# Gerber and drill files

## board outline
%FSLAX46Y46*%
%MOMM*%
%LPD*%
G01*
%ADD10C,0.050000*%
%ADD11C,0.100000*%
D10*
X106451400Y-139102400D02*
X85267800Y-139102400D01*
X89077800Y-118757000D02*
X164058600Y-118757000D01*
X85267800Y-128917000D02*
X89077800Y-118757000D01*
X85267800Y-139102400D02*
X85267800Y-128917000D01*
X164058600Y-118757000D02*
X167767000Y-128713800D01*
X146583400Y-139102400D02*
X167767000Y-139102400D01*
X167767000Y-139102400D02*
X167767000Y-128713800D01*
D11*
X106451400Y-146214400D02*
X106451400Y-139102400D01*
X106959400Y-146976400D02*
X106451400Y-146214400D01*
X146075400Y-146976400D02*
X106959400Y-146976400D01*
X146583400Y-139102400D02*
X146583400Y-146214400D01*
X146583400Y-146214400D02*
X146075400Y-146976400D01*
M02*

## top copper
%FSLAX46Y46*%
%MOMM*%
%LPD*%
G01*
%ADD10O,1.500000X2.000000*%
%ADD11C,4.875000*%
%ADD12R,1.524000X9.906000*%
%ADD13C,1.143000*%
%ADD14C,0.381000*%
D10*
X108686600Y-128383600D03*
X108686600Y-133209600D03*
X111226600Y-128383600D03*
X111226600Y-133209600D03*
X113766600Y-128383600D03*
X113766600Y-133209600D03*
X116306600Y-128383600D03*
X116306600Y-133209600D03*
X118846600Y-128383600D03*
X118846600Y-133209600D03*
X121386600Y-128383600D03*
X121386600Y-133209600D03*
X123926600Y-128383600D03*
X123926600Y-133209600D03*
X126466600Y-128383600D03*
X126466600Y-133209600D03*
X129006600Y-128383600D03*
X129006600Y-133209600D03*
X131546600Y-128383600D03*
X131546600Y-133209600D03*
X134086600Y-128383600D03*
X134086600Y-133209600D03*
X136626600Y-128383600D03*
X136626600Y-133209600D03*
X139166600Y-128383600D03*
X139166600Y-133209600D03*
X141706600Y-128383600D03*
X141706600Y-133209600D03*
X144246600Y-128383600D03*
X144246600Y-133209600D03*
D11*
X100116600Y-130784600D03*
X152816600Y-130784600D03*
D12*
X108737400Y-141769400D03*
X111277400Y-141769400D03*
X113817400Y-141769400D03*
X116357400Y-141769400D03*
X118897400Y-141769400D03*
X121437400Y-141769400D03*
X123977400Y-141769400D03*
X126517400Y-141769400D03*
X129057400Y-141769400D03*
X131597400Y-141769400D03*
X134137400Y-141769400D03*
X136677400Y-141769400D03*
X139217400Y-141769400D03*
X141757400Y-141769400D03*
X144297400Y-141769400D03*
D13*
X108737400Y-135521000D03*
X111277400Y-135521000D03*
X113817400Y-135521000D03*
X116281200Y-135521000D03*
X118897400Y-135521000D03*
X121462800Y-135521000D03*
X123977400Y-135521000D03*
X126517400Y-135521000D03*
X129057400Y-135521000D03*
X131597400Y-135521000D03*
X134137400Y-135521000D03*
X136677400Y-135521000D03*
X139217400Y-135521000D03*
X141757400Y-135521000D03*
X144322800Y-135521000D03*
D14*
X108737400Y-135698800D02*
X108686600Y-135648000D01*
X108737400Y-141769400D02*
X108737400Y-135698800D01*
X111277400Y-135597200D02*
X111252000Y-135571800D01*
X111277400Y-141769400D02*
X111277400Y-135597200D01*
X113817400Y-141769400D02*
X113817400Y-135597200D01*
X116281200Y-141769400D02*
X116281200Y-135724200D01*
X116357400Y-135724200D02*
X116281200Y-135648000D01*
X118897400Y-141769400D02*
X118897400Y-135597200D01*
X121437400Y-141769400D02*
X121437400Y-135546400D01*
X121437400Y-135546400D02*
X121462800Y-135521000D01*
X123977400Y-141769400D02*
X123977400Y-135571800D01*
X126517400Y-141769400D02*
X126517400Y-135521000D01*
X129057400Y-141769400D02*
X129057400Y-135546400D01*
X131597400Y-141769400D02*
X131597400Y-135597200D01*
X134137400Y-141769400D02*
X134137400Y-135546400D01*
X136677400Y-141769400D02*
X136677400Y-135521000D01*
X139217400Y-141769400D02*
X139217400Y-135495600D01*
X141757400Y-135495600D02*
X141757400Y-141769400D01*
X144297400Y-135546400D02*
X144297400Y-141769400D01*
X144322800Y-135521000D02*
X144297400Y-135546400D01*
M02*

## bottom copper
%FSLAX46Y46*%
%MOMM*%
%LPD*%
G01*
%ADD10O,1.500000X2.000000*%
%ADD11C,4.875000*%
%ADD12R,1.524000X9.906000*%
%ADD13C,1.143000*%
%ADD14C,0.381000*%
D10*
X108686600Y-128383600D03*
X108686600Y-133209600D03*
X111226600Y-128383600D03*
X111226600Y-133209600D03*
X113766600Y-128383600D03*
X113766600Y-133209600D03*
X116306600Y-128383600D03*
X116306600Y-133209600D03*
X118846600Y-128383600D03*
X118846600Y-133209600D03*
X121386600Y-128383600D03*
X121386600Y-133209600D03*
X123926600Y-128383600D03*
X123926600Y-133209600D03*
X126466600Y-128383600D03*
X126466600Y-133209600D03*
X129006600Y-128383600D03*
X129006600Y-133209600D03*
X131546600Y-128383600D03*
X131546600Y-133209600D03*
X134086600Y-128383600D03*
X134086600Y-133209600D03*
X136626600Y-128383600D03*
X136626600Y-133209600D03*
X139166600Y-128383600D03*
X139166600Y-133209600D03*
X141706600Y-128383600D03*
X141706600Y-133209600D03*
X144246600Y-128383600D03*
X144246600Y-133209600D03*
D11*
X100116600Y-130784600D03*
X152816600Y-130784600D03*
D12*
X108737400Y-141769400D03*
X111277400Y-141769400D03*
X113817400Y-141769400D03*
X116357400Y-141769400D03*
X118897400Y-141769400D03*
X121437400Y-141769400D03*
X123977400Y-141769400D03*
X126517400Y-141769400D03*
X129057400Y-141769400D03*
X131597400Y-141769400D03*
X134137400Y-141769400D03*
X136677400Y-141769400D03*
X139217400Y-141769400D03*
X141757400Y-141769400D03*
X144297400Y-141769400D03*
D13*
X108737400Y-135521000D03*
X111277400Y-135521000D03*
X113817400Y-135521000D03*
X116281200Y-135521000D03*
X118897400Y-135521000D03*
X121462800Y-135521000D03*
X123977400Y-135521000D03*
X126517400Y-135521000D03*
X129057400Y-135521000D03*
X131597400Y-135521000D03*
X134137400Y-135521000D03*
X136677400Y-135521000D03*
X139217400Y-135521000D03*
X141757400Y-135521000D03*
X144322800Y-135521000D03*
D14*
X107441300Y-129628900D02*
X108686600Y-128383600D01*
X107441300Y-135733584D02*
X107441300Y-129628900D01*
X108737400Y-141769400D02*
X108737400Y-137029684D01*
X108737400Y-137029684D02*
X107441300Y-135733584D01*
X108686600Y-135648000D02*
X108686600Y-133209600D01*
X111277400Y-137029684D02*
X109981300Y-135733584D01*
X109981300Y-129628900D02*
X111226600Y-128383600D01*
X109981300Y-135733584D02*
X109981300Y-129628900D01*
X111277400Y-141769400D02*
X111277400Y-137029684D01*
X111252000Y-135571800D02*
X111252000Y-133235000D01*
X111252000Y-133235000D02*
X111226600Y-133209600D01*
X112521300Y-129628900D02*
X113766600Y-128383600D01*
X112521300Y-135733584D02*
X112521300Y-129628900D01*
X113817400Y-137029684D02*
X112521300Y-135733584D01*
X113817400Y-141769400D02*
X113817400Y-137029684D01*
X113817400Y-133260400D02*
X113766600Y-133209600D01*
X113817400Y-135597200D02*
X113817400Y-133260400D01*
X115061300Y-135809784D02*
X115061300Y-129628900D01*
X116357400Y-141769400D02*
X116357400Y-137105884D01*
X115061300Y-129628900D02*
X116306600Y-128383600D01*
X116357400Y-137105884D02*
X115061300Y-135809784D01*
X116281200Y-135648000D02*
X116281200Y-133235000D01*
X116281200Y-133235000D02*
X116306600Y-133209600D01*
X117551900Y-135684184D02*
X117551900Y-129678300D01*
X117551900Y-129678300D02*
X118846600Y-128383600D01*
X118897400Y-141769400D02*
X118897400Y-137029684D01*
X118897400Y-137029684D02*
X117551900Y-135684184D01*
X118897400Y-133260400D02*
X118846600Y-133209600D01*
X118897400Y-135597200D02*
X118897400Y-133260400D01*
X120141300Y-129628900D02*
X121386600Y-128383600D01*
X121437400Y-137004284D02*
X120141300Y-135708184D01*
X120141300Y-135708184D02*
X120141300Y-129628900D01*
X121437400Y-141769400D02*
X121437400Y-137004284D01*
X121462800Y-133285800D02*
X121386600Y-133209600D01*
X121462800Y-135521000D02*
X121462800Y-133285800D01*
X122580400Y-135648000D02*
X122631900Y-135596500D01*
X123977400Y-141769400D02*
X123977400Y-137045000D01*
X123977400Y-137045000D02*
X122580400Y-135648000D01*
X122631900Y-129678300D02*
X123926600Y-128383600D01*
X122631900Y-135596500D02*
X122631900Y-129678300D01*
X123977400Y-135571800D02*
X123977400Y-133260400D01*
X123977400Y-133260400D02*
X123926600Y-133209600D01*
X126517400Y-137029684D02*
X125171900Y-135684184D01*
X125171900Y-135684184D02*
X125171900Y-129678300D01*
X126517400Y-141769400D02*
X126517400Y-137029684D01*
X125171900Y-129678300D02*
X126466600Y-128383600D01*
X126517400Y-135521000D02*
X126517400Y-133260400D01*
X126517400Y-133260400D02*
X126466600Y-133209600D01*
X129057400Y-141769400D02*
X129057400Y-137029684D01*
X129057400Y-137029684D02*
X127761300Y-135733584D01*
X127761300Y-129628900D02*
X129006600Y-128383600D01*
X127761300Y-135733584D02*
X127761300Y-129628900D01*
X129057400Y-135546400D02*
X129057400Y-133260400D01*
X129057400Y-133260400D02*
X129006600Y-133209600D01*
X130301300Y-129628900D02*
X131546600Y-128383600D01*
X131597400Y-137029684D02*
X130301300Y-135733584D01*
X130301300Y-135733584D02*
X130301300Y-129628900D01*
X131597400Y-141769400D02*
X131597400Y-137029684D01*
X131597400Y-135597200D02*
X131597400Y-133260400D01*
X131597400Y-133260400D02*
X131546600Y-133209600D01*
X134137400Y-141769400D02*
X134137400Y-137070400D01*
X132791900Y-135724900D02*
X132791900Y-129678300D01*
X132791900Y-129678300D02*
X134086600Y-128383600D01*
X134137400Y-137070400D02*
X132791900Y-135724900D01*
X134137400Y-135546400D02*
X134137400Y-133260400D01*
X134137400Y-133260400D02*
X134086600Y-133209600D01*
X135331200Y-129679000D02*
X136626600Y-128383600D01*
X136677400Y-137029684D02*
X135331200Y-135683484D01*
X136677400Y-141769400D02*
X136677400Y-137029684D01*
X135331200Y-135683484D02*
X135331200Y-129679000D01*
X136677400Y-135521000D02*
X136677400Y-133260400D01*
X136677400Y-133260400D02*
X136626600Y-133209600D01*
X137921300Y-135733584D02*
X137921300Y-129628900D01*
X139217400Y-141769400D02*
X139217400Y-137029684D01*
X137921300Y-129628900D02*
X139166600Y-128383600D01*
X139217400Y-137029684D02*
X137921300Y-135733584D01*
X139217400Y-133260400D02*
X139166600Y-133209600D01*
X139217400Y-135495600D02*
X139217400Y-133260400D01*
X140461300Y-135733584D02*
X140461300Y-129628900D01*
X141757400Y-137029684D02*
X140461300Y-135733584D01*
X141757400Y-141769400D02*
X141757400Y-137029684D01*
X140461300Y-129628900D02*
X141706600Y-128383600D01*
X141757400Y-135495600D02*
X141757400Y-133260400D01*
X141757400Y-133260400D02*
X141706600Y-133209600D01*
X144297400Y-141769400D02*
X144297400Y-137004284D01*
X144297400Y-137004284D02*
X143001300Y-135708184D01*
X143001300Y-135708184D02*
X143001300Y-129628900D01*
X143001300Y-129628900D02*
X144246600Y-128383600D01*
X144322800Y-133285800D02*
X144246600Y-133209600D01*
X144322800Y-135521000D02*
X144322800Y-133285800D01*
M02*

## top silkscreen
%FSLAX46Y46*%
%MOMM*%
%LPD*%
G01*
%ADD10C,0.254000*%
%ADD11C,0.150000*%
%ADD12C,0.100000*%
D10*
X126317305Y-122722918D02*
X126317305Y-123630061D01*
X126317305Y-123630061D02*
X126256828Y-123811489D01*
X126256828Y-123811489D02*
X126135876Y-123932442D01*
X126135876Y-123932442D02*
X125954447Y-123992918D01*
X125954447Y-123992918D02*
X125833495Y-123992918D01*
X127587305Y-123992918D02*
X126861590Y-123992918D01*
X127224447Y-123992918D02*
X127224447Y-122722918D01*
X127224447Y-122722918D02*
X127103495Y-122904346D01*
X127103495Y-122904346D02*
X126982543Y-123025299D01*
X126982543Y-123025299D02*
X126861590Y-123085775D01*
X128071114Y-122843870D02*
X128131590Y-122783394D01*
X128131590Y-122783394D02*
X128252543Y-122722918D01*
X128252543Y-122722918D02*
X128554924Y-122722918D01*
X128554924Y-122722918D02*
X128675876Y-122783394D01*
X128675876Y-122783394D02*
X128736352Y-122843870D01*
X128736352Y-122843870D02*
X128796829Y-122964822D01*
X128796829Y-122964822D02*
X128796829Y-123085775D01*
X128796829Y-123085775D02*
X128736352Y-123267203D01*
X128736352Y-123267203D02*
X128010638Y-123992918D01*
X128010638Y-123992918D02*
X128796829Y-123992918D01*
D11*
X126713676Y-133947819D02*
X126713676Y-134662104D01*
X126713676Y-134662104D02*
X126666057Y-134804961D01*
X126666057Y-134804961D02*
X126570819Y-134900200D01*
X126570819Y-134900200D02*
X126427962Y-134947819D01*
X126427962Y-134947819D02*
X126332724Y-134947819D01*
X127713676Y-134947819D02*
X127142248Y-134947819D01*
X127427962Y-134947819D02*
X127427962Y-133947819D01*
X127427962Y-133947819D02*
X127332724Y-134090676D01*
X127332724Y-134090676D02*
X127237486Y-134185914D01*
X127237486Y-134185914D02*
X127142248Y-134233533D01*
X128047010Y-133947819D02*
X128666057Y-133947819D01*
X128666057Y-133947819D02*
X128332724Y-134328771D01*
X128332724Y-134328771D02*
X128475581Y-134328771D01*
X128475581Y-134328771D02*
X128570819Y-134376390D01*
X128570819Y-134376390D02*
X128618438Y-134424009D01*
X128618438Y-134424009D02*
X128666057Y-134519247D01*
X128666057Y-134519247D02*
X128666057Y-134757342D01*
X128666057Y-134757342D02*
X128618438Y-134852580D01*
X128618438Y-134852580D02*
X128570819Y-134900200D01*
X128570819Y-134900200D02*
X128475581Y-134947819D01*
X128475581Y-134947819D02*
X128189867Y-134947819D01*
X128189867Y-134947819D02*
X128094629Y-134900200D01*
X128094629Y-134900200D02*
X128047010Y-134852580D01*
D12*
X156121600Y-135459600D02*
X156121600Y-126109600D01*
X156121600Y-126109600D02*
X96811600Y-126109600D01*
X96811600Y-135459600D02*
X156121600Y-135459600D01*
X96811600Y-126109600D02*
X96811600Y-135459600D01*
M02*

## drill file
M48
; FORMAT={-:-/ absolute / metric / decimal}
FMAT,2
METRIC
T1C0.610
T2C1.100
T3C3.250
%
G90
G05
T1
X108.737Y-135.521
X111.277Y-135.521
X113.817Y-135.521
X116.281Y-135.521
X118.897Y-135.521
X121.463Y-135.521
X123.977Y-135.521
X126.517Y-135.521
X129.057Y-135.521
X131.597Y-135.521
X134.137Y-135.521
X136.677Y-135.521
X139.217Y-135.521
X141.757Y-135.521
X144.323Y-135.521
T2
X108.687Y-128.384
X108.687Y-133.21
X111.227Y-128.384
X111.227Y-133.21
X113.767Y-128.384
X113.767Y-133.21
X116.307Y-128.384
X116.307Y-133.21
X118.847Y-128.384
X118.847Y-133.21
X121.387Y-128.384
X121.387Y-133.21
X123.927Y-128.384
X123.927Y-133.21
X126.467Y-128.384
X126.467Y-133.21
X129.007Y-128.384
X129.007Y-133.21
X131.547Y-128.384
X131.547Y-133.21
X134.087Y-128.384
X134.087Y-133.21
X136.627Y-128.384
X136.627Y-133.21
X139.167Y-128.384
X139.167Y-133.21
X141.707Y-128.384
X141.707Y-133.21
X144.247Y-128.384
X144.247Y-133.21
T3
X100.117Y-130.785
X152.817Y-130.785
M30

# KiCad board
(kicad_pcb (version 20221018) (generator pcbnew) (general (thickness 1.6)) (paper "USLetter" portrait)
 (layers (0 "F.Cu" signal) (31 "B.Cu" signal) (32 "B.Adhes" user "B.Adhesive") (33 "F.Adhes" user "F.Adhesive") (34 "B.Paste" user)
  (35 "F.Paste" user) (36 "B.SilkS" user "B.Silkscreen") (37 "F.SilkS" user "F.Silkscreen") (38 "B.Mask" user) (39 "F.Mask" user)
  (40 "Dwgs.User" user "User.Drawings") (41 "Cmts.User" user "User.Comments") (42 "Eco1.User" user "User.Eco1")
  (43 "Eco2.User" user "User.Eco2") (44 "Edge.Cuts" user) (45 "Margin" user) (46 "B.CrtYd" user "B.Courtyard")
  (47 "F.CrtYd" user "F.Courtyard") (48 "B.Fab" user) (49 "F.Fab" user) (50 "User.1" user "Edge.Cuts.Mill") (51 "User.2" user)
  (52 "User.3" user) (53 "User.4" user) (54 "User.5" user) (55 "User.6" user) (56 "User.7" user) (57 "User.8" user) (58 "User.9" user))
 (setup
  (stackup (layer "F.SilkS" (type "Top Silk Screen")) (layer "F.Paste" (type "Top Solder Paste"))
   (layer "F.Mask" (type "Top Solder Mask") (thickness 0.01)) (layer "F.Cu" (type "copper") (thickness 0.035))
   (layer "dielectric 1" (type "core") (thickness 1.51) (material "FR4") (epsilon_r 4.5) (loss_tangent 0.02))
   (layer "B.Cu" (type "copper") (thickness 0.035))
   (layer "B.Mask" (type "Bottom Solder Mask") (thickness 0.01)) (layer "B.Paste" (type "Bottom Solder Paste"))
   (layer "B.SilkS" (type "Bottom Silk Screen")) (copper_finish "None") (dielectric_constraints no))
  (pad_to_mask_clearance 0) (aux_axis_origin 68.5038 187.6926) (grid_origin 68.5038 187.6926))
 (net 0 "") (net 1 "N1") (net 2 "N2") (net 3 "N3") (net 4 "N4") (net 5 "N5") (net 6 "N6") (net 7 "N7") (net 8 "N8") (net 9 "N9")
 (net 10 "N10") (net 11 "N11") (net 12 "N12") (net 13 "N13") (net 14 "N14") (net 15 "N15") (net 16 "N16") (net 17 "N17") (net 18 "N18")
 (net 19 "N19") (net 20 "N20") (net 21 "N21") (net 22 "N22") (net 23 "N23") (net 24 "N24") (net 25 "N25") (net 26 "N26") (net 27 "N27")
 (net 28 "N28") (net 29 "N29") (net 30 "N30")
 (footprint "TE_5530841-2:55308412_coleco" (layer "F.Cu") (at 108.6866 133.2096 180)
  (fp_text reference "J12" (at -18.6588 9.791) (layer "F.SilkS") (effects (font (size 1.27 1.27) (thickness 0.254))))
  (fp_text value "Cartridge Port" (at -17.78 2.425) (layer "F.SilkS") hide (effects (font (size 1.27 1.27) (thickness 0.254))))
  (fp_line (start -47.435 -2.25) (end -47.435 7.1) (stroke (width 0.1) (type solid)) (layer "F.SilkS"))
  (fp_line (start -47.435 7.1) (end 11.875 7.1) (stroke (width 0.1) (type solid)) (layer "F.SilkS"))
  (fp_line (start 11.875 -2.25) (end -47.435 -2.25) (stroke (width 0.1) (type solid)) (layer "F.SilkS"))
  (fp_line (start 11.875 7.1) (end 11.875 -2.25) (stroke (width 0.1) (type solid)) (layer "F.SilkS"))
  (pad "1" thru_hole oval (at 0 4.826 180) (size 1.5 2) (drill 1.1) (layers "*.Cu" "*.Mask") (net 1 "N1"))
  (pad "2" thru_hole oval (at 0 0 180) (size 1.5 2) (drill 1.1) (layers "*.Cu" "*.Mask") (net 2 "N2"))
  (pad "3" thru_hole oval (at -2.54 4.826 180) (size 1.5 2) (drill 1.1) (layers "*.Cu" "*.Mask") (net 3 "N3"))
  (pad "4" thru_hole oval (at -2.54 0 180) (size 1.5 2) (drill 1.1) (layers "*.Cu" "*.Mask") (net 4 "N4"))
  (pad "5" thru_hole oval (at -5.08 4.826 180) (size 1.5 2) (drill 1.1) (layers "*.Cu" "*.Mask") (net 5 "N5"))
  (pad "6" thru_hole oval (at -5.08 0 180) (size 1.5 2) (drill 1.1) (layers "*.Cu" "*.Mask") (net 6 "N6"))
  (pad "7" thru_hole oval (at -7.62 4.826 180) (size 1.5 2) (drill 1.1) (layers "*.Cu" "*.Mask") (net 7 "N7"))
  (pad "8" thru_hole oval (at -7.62 0 180) (size 1.5 2) (drill 1.1) (layers "*.Cu" "*.Mask") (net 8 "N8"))
  (pad "9" thru_hole oval (at -10.16 4.826 180) (size 1.5 2) (drill 1.1) (layers "*.Cu" "*.Mask") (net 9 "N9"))
  (pad "10" thru_hole oval (at -10.16 0 180) (size 1.5 2) (drill 1.1) (layers "*.Cu" "*.Mask") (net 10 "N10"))
  (pad "11" thru_hole oval (at -12.7 4.826 180) (size 1.5 2) (drill 1.1) (layers "*.Cu" "*.Mask") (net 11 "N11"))
  (pad "12" thru_hole oval (at -12.7 0 180) (size 1.5 2) (drill 1.1) (layers "*.Cu" "*.Mask") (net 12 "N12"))
  (pad "13" thru_hole oval (at -15.24 4.826 180) (size 1.5 2) (drill 1.1) (layers "*.Cu" "*.Mask") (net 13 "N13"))
  (pad "14" thru_hole oval (at -15.24 0 180) (size 1.5 2) (drill 1.1) (layers "*.Cu" "*.Mask") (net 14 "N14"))
  (pad "15" thru_hole oval (at -17.78 4.826 180) (size 1.5 2) (drill 1.1) (layers "*.Cu" "*.Mask") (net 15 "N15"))
  (pad "16" thru_hole oval (at -17.78 0 180) (size 1.5 2) (drill 1.1) (layers "*.Cu" "*.Mask") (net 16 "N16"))
  (pad "17" thru_hole oval (at -20.32 4.826 180) (size 1.5 2) (drill 1.1) (layers "*.Cu" "*.Mask") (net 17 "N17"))
  (pad "18" thru_hole oval (at -20.32 0 180) (size 1.5 2) (drill 1.1) (layers "*.Cu" "*.Mask") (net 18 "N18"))
  (pad "19" thru_hole oval (at -22.86 4.826 180) (size 1.5 2) (drill 1.1) (layers "*.Cu" "*.Mask") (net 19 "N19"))
  (pad "20" thru_hole oval (at -22.86 0 180) (size 1.5 2) (drill 1.1) (layers "*.Cu" "*.Mask") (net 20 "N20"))
  (pad "21" thru_hole oval (at -25.4 4.826 180) (size 1.5 2) (drill 1.1) (layers "*.Cu" "*.Mask") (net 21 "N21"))
  (pad "22" thru_hole oval (at -25.4 0 180) (size 1.5 2) (drill 1.1) (layers "*.Cu" "*.Mask") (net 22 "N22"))
  (pad "23" thru_hole oval (at -27.94 4.826 180) (size 1.5 2) (drill 1.1) (layers "*.Cu" "*.Mask") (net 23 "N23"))
  (pad "24" thru_hole oval (at -27.94 0 180) (size 1.5 2) (drill 1.1) (layers "*.Cu" "*.Mask") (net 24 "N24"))
  (pad "25" thru_hole oval (at -30.48 4.826 180) (size 1.5 2) (drill 1.1) (layers "*.Cu" "*.Mask") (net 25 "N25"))
  (pad "26" thru_hole oval (at -30.48 0 180) (size 1.5 2) (drill 1.1) (layers "*.Cu" "*.Mask") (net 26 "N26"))
  (pad "27" thru_hole oval (at -33.02 4.826 180) (size 1.5 2) (drill 1.1) (layers "*.Cu" "*.Mask") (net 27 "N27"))
  (pad "28" thru_hole oval (at -33.02 0 180) (size 1.5 2) (drill 1.1) (layers "*.Cu" "*.Mask") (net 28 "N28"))
  (pad "29" thru_hole oval (at -35.56 4.826 180) (size 1.5 2) (drill 1.1) (layers "*.Cu" "*.Mask") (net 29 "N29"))
  (pad "30" thru_hole oval (at -35.56 0 180) (size 1.5 2) (drill 1.1) (layers "*.Cu" "*.Mask") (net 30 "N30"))
  (pad "MH1" thru_hole circle (at 8.57 2.425 180) (size 4.875 4.875) (drill 3.25) (layers "*.Cu" "*.Mask"))
  (pad "MH2" thru_hole circle (at -44.13 2.425 180) (size 4.875 4.875) (drill 3.25) (layers "*.Cu" "*.Mask")))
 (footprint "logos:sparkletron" (layer "F.Cu") (at 138.3842 226.960062)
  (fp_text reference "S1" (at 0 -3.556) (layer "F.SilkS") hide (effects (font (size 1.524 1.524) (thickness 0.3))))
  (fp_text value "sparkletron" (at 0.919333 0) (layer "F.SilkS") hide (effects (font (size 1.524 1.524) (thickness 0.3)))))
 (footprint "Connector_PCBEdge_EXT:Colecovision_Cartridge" (layer "F.Cu") (at 104.9274 143.6744)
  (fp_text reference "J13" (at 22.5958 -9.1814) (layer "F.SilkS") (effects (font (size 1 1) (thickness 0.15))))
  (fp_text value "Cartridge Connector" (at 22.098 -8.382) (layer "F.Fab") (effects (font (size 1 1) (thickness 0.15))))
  (fp_line (start 1.524 2.54) (end 1.524 -4.572) (stroke (width 0.1) (type solid)) (layer "Edge.Cuts"))
  (fp_line (start 2.032 3.302) (end 1.524 2.54) (stroke (width 0.1) (type solid)) (layer "Edge.Cuts"))
  (fp_line (start 41.148 3.302) (end 2.032 3.302) (stroke (width 0.1) (type solid)) (layer "Edge.Cuts"))
  (fp_line (start 41.656 -4.572) (end 41.656 2.54) (stroke (width 0.1) (type solid)) (layer "Edge.Cuts"))
  (fp_line (start 41.656 2.54) (end 41.148 3.302) (stroke (width 0.1) (type solid)) (layer "Edge.Cuts"))
  (pad "1" connect rect (at 3.81 -1.905) (size 1.524 9.906) (layers "B.Cu" "B.Mask") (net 1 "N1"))
  (pad "2" connect rect (at 3.81 -1.905) (size 1.524 9.906) (layers "F.Cu" "F.Mask") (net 2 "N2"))
  (pad "3" connect rect (at 6.35 -1.905) (size 1.524 9.906) (layers "B.Cu" "B.Mask") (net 3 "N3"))
  (pad "4" connect rect (at 6.35 -1.905) (size 1.524 9.906) (layers "F.Cu" "F.Mask") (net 4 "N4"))
  (pad "5" connect rect (at 8.89 -1.905) (size 1.524 9.906) (layers "B.Cu" "B.Mask") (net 5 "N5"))
  (pad "6" connect rect (at 8.89 -1.905) (size 1.524 9.906) (layers "F.Cu" "F.Mask") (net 6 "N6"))
  (pad "7" connect rect (at 11.43 -1.905) (size 1.524 9.906) (layers "B.Cu" "B.Mask") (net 7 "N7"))
  (pad "8" connect rect (at 11.43 -1.905) (size 1.524 9.906) (layers "F.Cu" "F.Mask") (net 8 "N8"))
  (pad "9" connect rect (at 13.97 -1.905) (size 1.524 9.906) (layers "B.Cu" "B.Mask") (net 9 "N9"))
  (pad "10" connect rect (at 13.97 -1.905) (size 1.524 9.906) (layers "F.Cu" "F.Mask") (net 10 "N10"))
  (pad "11" connect rect (at 16.51 -1.905) (size 1.524 9.906) (layers "B.Cu" "B.Mask") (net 11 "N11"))
  (pad "12" connect rect (at 16.51 -1.905) (size 1.524 9.906) (layers "F.Cu" "F.Mask") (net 12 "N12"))
  (pad "13" connect rect (at 19.05 -1.905) (size 1.524 9.906) (layers "B.Cu" "B.Mask") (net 13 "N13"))
  (pad "14" connect rect (at 19.05 -1.905) (size 1.524 9.906) (layers "F.Cu" "F.Mask") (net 14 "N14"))
  (pad "15" connect rect (at 21.59 -1.905) (size 1.524 9.906) (layers "B.Cu" "B.Mask") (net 15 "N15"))
  (pad "16" connect rect (at 21.59 -1.905) (size 1.524 9.906) (layers "F.Cu" "F.Mask") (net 16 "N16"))
  (pad "17" connect rect (at 24.13 -1.905) (size 1.524 9.906) (layers "B.Cu" "B.Mask") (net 17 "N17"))
  (pad "18" connect rect (at 24.13 -1.905) (size 1.524 9.906) (layers "F.Cu" "F.Mask") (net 18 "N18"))
  (pad "19" connect rect (at 26.67 -1.905) (size 1.524 9.906) (layers "B.Cu" "B.Mask") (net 19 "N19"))
  (pad "20" connect rect (at 26.67 -1.905) (size 1.524 9.906) (layers "F.Cu" "F.Mask") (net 20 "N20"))
  (pad "21" connect rect (at 29.21 -1.905) (size 1.524 9.906) (layers "B.Cu" "B.Mask") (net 21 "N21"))
  (pad "22" connect rect (at 29.21 -1.905) (size 1.524 9.906) (layers "F.Cu" "F.Mask") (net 22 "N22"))
  (pad "23" connect rect (at 31.75 -1.905) (size 1.524 9.906) (layers "B.Cu" "B.Mask") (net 23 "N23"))
  (pad "24" connect rect (at 31.75 -1.905) (size 1.524 9.906) (layers "F.Cu" "F.Mask") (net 24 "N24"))
  (pad "25" connect rect (at 34.29 -1.905) (size 1.524 9.906) (layers "B.Cu" "B.Mask") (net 25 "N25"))
  (pad "26" connect rect (at 34.29 -1.905) (size 1.524 9.906) (layers "F.Cu" "F.Mask") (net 26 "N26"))
  (pad "27" connect rect (at 36.83 -1.905) (size 1.524 9.906) (layers "B.Cu" "B.Mask") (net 27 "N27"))
  (pad "28" connect rect (at 36.83 -1.905) (size 1.524 9.906) (layers "F.Cu" "F.Mask") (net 28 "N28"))
  (pad "29" connect rect (at 39.37 -1.905) (size 1.524 9.906) (layers "B.Cu" "B.Mask") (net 29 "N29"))
  (pad "30" connect rect (at 39.37 -1.905) (size 1.524 9.906) (layers "F.Cu" "F.Mask") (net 30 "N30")))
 (gr_line (start 106.4514 139.1024) (end 85.2678 139.1024) (stroke (width 0.05) (type default)) (layer "Edge.Cuts"))
 (gr_line (start 89.0778 118.757) (end 164.0586 118.757) (stroke (width 0.05) (type default)) (layer "Edge.Cuts"))
 (gr_line (start 85.2678 128.917) (end 89.0778 118.757) (stroke (width 0.05) (type default)) (layer "Edge.Cuts"))
 (gr_line (start 85.2678 139.1024) (end 85.2678 128.917) (stroke (width 0.05) (type default)) (layer "Edge.Cuts"))
 (gr_line (start 164.0586 118.757) (end 167.767 128.7138) (stroke (width 0.05) (type default)) (layer "Edge.Cuts"))
 (gr_line (start 146.5834 139.1024) (end 167.767 139.1024) (stroke (width 0.05) (type default)) (layer "Edge.Cuts"))
 (gr_line (start 167.767 139.1024) (end 167.767 128.7138) (stroke (width 0.05) (type default)) (layer "Edge.Cuts"))
 (segment (start 107.4413 129.6289) (end 108.6866 128.3836) (width 0.381) (layer "B.Cu") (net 1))
 (segment (start 107.4413 135.733584) (end 107.4413 129.6289) (width 0.381) (layer "B.Cu") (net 1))
 (segment (start 108.7374 141.7694) (end 108.7374 137.029684) (width 0.381) (layer "B.Cu") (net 1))
 (segment (start 108.7374 137.029684) (end 107.4413 135.733584) (width 0.381) (layer "B.Cu") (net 1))
 (segment (start 108.7374 135.6988) (end 108.6866 135.648) (width 0.381) (layer "F.Cu") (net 2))
 (segment (start 108.7374 141.7694) (end 108.7374 135.6988) (width 0.381) (layer "F.Cu") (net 2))
 (via (at 108.7374 135.521) (size 1.143) (drill 0.6096) (layers "F.Cu" "B.Cu") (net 2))
 (segment (start 108.6866 135.648) (end 108.6866 133.2096) (width 0.381) (layer "B.Cu") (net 2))
 (segment (start 111.2774 137.029684) (end 109.9813 135.733584) (width 0.381) (layer "B.Cu") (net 3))
 (segment (start 109.9813 129.6289) (end 111.2266 128.3836) (width 0.381) (layer "B.Cu") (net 3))
 (segment (start 109.9813 135.733584) (end 109.9813 129.6289) (width 0.381) (layer "B.Cu") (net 3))
 (segment (start 111.2774 141.7694) (end 111.2774 137.029684) (width 0.381) (layer "B.Cu") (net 3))
 (segment (start 111.2774 135.5972) (end 111.252 135.5718) (width 0.381) (layer "F.Cu") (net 4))
 (segment (start 111.2774 141.7694) (end 111.2774 135.5972) (width 0.381) (layer "F.Cu") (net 4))
 (via (at 111.2774 135.521) (size 1.143) (drill 0.6096) (layers "F.Cu" "B.Cu") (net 4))
 (segment (start 111.252 135.5718) (end 111.252 133.235) (width 0.381) (layer "B.Cu") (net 4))
 (segment (start 111.252 133.235) (end 111.2266 133.2096) (width 0.381) (layer "B.Cu") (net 4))
 (segment (start 112.5213 129.6289) (end 113.7666 128.3836) (width 0.381) (layer "B.Cu") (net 5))
 (segment (start 112.5213 135.733584) (end 112.5213 129.6289) (width 0.381) (layer "B.Cu") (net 5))
 (segment (start 113.8174 137.029684) (end 112.5213 135.733584) (width 0.381) (layer "B.Cu") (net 5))
 (segment (start 113.8174 141.7694) (end 113.8174 137.029684) (width 0.381) (layer "B.Cu") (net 5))
 (segment (start 113.8174 141.7694) (end 113.8174 135.5972) (width 0.381) (layer "F.Cu") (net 6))
 (via (at 113.8174 135.521) (size 1.143) (drill 0.6096) (layers "F.Cu" "B.Cu") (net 6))
 (segment (start 113.8174 133.2604) (end 113.7666 133.2096) (width 0.381) (layer "B.Cu") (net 6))
 (segment (start 113.8174 135.5972) (end 113.8174 133.2604) (width 0.381) (layer "B.Cu") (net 6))
 (segment (start 115.0613 135.809784) (end 115.0613 129.6289) (width 0.381) (layer "B.Cu") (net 7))
 (segment (start 116.3574 141.7694) (end 116.3574 137.105884) (width 0.381) (layer "B.Cu") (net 7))
 (segment (start 115.0613 129.6289) (end 116.3066 128.3836) (width 0.381) (layer "B.Cu") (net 7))
 (segment (start 116.3574 137.105884) (end 115.0613 135.809784) (width 0.381) (layer "B.Cu") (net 7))
 (segment (start 116.2812 141.7694) (end 116.2812 135.7242) (width 0.381) (layer "F.Cu") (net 8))
 (segment (start 116.3574 135.7242) (end 116.2812 135.648) (width 0.381) (layer "F.Cu") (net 8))
 (via (at 116.2812 135.521) (size 1.143) (drill 0.6096) (layers "F.Cu" "B.Cu") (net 8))
 (segment (start 116.2812 135.648) (end 116.2812 133.235) (width 0.381) (layer "B.Cu") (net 8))
 (segment (start 116.2812 133.235) (end 116.3066 133.2096) (width 0.381) (layer "B.Cu") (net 8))
 (segment (start 117.5519 135.684184) (end 117.5519 129.6783) (width 0.381) (layer "B.Cu") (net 9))
 (segment (start 117.5519 129.6783) (end 118.8466 128.3836) (width 0.381) (layer "B.Cu") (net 9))
 (segment (start 118.8974 141.7694) (end 118.8974 137.029684) (width 0.381) (layer "B.Cu") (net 9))
 (segment (start 118.8974 137.029684) (end 117.5519 135.684184) (width 0.381) (layer "B.Cu") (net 9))
 (segment (start 118.8974 141.7694) (end 118.8974 135.5972) (width 0.381) (layer "F.Cu") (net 10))
 (via (at 118.8974 135.521) (size 1.143) (drill 0.6096) (layers "F.Cu" "B.Cu") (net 10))
 (segment (start 118.8974 133.2604) (end 118.8466 133.2096) (width 0.381) (layer "B.Cu") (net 10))
 (segment (start 118.8974 135.5972) (end 118.8974 133.2604) (width 0.381) (layer "B.Cu") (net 10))
 (segment (start 120.1413 129.6289) (end 121.3866 128.3836) (width 0.381) (layer "B.Cu") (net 11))
 (segment (start 121.4374 137.004284) (end 120.1413 135.708184) (width 0.381) (layer "B.Cu") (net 11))
 (segment (start 120.1413 135.708184) (end 120.1413 129.6289) (width 0.381) (layer "B.Cu") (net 11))
 (segment (start 121.4374 141.7694) (end 121.4374 137.004284) (width 0.381) (layer "B.Cu") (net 11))
 (segment (start 121.4374 141.7694) (end 121.4374 135.5464) (width 0.381) (layer "F.Cu") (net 12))
 (segment (start 121.4374 135.5464) (end 121.4628 135.521) (width 0.381) (layer "F.Cu") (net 12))
 (via (at 121.4628 135.521) (size 1.143) (drill 0.6096) (layers "F.Cu" "B.Cu") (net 12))
 (segment (start 121.4628 133.2858) (end 121.3866 133.2096) (width 0.381) (layer "B.Cu") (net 12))
 (segment (start 121.4628 135.521) (end 121.4628 133.2858) (width 0.381) (layer "B.Cu") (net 12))
 (segment (start 122.5804 135.648) (end 122.6319 135.5965) (width 0.381) (layer "B.Cu") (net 13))
 (segment (start 123.9774 141.7694) (end 123.9774 137.045) (width 0.381) (layer "B.Cu") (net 13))
 (segment (start 123.9774 137.045) (end 122.5804 135.648) (width 0.381) (layer "B.Cu") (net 13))
 (segment (start 122.6319 129.6783) (end 123.9266 128.3836) (width 0.381) (layer "B.Cu") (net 13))
 (segment (start 122.6319 135.5965) (end 122.6319 129.6783) (width 0.381) (layer "B.Cu") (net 13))
 (segment (start 123.9774 141.7694) (end 123.9774 135.5718) (width 0.381) (layer "F.Cu") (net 14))
 (via (at 123.9774 135.521) (size 1.143) (drill 0.6096) (layers "F.Cu" "B.Cu") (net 14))
 (segment (start 123.9774 135.5718) (end 123.9774 133.2604) (width 0.381) (layer "B.Cu") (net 14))
 (segment (start 123.9774 133.2604) (end 123.9266 133.2096) (width 0.381) (layer "B.Cu") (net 14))
 (segment (start 126.5174 137.029684) (end 125.1719 135.684184) (width 0.381) (layer "B.Cu") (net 15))
 (segment (start 125.1719 135.684184) (end 125.1719 129.6783) (width 0.381) (layer "B.Cu") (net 15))
 (segment (start 126.5174 141.7694) (end 126.5174 137.029684) (width 0.381) (layer "B.Cu") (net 15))
 (segment (start 125.1719 129.6783) (end 126.4666 128.3836) (width 0.381) (layer "B.Cu") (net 15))
 (segment (start 126.5174 141.7694) (end 126.5174 135.521) (width 0.381) (layer "F.Cu") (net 16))
 (via (at 126.5174 135.521) (size 1.143) (drill 0.6096) (layers "F.Cu" "B.Cu") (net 16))
 (segment (start 126.5174 135.521) (end 126.5174 133.2604) (width 0.381) (layer "B.Cu") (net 16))
 (segment (start 126.5174 133.2604) (end 126.4666 133.2096) (width 0.381) (layer "B.Cu") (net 16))
 (segment (start 129.0574 141.7694) (end 129.0574 137.029684) (width 0.381) (layer "B.Cu") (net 17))
 (segment (start 129.0574 137.029684) (end 127.7613 135.733584) (width 0.381) (layer "B.Cu") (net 17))
 (segment (start 127.7613 129.6289) (end 129.0066 128.3836) (width 0.381) (layer "B.Cu") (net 17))
 (segment (start 127.7613 135.733584) (end 127.7613 129.6289) (width 0.381) (layer "B.Cu") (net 17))
 (segment (start 129.0574 141.7694) (end 129.0574 135.5464) (width 0.381) (layer "F.Cu") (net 18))
 (via (at 129.0574 135.521) (size 1.143) (drill 0.6096) (layers "F.Cu" "B.Cu") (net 18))
 (segment (start 129.0574 135.5464) (end 129.0574 133.2604) (width 0.381) (layer "B.Cu") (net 18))
 (segment (start 129.0574 133.2604) (end 129.0066 133.2096) (width 0.381) (layer "B.Cu") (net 18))
 (segment (start 130.3013 129.6289) (end 131.5466 128.3836) (width 0.381) (layer "B.Cu") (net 19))
 (segment (start 131.5974 137.029684) (end 130.3013 135.733584) (width 0.381) (layer "B.Cu") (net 19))
 (segment (start 130.3013 135.733584) (end 130.3013 129.6289) (width 0.381) (layer "B.Cu") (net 19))
 (segment (start 131.5974 141.7694) (end 131.5974 137.029684) (width 0.381) (layer "B.Cu") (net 19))
 (segment (start 131.5974 141.7694) (end 131.5974 135.5972) (width 0.381) (layer "F.Cu") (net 20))
 (via (at 131.5974 135.521) (size 1.143) (drill 0.6096) (layers "F.Cu" "B.Cu") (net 20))
 (segment (start 131.5974 135.5972) (end 131.5974 133.2604) (width 0.381) (layer "B.Cu") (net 20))
 (segment (start 131.5974 133.2604) (end 131.5466 133.2096) (width 0.381) (layer "B.Cu") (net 20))
 (segment (start 134.1374 141.7694) (end 134.1374 137.0704) (width 0.381) (layer "B.Cu") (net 21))
 (segment (start 132.7919 135.7249) (end 132.7919 129.6783) (width 0.381) (layer "B.Cu") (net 21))
 (segment (start 132.7919 129.6783) (end 134.0866 128.3836) (width 0.381) (layer "B.Cu") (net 21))
 (segment (start 134.1374 137.0704) (end 132.7919 135.7249) (width 0.381) (layer "B.Cu") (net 21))
 (segment (start 134.1374 141.7694) (end 134.1374 135.5464) (width 0.381) (layer "F.Cu") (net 22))
 (via (at 134.1374 135.521) (size 1.143) (drill 0.6096) (layers "F.Cu" "B.Cu") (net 22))
 (segment (start 134.1374 135.5464) (end 134.1374 133.2604) (width 0.381) (layer "B.Cu") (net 22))
 (segment (start 134.1374 133.2604) (end 134.0866 133.2096) (width 0.381) (layer "B.Cu") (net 22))
 (segment (start 135.3312 129.679) (end 136.6266 128.3836) (width 0.381) (layer "B.Cu") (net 23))
 (segment (start 136.6774 137.029684) (end 135.3312 135.683484) (width 0.381) (layer "B.Cu") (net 23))
 (segment (start 136.6774 141.7694) (end 136.6774 137.029684) (width 0.381) (layer "B.Cu") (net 23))
 (segment (start 135.3312 135.683484) (end 135.3312 129.679) (width 0.381) (layer "B.Cu") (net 23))
 (segment (start 136.6774 141.7694) (end 136.6774 135.521) (width 0.381) (layer "F.Cu") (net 24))
 (via (at 136.6774 135.521) (size 1.143) (drill 0.6096) (layers "F.Cu" "B.Cu") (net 24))
 (segment (start 136.6774 135.521) (end 136.6774 133.2604) (width 0.381) (layer "B.Cu") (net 24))
 (segment (start 136.6774 133.2604) (end 136.6266 133.2096) (width 0.381) (layer "B.Cu") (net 24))
 (segment (start 137.9213 135.733584) (end 137.9213 129.6289) (width 0.381) (layer "B.Cu") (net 25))
 (segment (start 139.2174 141.7694) (end 139.2174 137.029684) (width 0.381) (layer "B.Cu") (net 25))
 (segment (start 137.9213 129.6289) (end 139.1666 128.3836) (width 0.381) (layer "B.Cu") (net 25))
 (segment (start 139.2174 137.029684) (end 137.9213 135.733584) (width 0.381) (layer "B.Cu") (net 25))
 (segment (start 139.2174 141.7694) (end 139.2174 135.4956) (width 0.381) (layer "F.Cu") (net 26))
 (via (at 139.2174 135.521) (size 1.143) (drill 0.6096) (layers "F.Cu" "B.Cu") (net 26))
 (segment (start 139.2174 133.2604) (end 139.1666 133.2096) (width 0.381) (layer "B.Cu") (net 26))
 (segment (start 139.2174 135.4956) (end 139.2174 133.2604) (width 0.381) (layer "B.Cu") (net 26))
 (segment (start 140.4613 135.733584) (end 140.4613 129.6289) (width 0.381) (layer "B.Cu") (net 27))
 (segment (start 141.7574 137.029684) (end 140.4613 135.733584) (width 0.381) (layer "B.Cu") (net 27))
 (segment (start 141.7574 141.7694) (end 141.7574 137.029684) (width 0.381) (layer "B.Cu") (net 27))
 (segment (start 140.4613 129.6289) (end 141.7066 128.3836) (width 0.381) (layer "B.Cu") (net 27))
 (segment (start 141.7574 135.4956) (end 141.7574 141.7694) (width 0.381) (layer "F.Cu") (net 28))
 (via (at 141.7574 135.521) (size 1.143) (drill 0.6096) (layers "F.Cu" "B.Cu") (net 28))
 (segment (start 141.7574 135.4956) (end 141.7574 133.2604) (width 0.381) (layer "B.Cu") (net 28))
 (segment (start 141.7574 133.2604) (end 141.7066 133.2096) (width 0.381) (layer "B.Cu") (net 28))
 (segment (start 144.2974 141.7694) (end 144.2974 137.004284) (width 0.381) (layer "B.Cu") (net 29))
 (segment (start 144.2974 137.004284) (end 143.0013 135.708184) (width 0.381) (layer "B.Cu") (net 29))
 (segment (start 143.0013 135.708184) (end 143.0013 129.6289) (width 0.381) (layer "B.Cu") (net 29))
 (segment (start 143.0013 129.6289) (end 144.2466 128.3836) (width 0.381) (layer "B.Cu") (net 29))
 (segment (start 144.2974 135.5464) (end 144.2974 141.7694) (width 0.381) (layer "F.Cu") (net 30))
 (segment (start 144.3228 135.521) (end 144.2974 135.5464) (width 0.381) (layer "F.Cu") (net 30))
 (via (at 144.3228 135.521) (size 1.143) (drill 0.6096) (layers "F.Cu" "B.Cu") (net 30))
 (segment (start 144.3228 133.2858) (end 144.2466 133.2096) (width 0.381) (layer "B.Cu") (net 30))
 (segment (start 144.3228 135.521) (end 144.3228 133.2858) (width 0.381) (layer "B.Cu") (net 30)))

